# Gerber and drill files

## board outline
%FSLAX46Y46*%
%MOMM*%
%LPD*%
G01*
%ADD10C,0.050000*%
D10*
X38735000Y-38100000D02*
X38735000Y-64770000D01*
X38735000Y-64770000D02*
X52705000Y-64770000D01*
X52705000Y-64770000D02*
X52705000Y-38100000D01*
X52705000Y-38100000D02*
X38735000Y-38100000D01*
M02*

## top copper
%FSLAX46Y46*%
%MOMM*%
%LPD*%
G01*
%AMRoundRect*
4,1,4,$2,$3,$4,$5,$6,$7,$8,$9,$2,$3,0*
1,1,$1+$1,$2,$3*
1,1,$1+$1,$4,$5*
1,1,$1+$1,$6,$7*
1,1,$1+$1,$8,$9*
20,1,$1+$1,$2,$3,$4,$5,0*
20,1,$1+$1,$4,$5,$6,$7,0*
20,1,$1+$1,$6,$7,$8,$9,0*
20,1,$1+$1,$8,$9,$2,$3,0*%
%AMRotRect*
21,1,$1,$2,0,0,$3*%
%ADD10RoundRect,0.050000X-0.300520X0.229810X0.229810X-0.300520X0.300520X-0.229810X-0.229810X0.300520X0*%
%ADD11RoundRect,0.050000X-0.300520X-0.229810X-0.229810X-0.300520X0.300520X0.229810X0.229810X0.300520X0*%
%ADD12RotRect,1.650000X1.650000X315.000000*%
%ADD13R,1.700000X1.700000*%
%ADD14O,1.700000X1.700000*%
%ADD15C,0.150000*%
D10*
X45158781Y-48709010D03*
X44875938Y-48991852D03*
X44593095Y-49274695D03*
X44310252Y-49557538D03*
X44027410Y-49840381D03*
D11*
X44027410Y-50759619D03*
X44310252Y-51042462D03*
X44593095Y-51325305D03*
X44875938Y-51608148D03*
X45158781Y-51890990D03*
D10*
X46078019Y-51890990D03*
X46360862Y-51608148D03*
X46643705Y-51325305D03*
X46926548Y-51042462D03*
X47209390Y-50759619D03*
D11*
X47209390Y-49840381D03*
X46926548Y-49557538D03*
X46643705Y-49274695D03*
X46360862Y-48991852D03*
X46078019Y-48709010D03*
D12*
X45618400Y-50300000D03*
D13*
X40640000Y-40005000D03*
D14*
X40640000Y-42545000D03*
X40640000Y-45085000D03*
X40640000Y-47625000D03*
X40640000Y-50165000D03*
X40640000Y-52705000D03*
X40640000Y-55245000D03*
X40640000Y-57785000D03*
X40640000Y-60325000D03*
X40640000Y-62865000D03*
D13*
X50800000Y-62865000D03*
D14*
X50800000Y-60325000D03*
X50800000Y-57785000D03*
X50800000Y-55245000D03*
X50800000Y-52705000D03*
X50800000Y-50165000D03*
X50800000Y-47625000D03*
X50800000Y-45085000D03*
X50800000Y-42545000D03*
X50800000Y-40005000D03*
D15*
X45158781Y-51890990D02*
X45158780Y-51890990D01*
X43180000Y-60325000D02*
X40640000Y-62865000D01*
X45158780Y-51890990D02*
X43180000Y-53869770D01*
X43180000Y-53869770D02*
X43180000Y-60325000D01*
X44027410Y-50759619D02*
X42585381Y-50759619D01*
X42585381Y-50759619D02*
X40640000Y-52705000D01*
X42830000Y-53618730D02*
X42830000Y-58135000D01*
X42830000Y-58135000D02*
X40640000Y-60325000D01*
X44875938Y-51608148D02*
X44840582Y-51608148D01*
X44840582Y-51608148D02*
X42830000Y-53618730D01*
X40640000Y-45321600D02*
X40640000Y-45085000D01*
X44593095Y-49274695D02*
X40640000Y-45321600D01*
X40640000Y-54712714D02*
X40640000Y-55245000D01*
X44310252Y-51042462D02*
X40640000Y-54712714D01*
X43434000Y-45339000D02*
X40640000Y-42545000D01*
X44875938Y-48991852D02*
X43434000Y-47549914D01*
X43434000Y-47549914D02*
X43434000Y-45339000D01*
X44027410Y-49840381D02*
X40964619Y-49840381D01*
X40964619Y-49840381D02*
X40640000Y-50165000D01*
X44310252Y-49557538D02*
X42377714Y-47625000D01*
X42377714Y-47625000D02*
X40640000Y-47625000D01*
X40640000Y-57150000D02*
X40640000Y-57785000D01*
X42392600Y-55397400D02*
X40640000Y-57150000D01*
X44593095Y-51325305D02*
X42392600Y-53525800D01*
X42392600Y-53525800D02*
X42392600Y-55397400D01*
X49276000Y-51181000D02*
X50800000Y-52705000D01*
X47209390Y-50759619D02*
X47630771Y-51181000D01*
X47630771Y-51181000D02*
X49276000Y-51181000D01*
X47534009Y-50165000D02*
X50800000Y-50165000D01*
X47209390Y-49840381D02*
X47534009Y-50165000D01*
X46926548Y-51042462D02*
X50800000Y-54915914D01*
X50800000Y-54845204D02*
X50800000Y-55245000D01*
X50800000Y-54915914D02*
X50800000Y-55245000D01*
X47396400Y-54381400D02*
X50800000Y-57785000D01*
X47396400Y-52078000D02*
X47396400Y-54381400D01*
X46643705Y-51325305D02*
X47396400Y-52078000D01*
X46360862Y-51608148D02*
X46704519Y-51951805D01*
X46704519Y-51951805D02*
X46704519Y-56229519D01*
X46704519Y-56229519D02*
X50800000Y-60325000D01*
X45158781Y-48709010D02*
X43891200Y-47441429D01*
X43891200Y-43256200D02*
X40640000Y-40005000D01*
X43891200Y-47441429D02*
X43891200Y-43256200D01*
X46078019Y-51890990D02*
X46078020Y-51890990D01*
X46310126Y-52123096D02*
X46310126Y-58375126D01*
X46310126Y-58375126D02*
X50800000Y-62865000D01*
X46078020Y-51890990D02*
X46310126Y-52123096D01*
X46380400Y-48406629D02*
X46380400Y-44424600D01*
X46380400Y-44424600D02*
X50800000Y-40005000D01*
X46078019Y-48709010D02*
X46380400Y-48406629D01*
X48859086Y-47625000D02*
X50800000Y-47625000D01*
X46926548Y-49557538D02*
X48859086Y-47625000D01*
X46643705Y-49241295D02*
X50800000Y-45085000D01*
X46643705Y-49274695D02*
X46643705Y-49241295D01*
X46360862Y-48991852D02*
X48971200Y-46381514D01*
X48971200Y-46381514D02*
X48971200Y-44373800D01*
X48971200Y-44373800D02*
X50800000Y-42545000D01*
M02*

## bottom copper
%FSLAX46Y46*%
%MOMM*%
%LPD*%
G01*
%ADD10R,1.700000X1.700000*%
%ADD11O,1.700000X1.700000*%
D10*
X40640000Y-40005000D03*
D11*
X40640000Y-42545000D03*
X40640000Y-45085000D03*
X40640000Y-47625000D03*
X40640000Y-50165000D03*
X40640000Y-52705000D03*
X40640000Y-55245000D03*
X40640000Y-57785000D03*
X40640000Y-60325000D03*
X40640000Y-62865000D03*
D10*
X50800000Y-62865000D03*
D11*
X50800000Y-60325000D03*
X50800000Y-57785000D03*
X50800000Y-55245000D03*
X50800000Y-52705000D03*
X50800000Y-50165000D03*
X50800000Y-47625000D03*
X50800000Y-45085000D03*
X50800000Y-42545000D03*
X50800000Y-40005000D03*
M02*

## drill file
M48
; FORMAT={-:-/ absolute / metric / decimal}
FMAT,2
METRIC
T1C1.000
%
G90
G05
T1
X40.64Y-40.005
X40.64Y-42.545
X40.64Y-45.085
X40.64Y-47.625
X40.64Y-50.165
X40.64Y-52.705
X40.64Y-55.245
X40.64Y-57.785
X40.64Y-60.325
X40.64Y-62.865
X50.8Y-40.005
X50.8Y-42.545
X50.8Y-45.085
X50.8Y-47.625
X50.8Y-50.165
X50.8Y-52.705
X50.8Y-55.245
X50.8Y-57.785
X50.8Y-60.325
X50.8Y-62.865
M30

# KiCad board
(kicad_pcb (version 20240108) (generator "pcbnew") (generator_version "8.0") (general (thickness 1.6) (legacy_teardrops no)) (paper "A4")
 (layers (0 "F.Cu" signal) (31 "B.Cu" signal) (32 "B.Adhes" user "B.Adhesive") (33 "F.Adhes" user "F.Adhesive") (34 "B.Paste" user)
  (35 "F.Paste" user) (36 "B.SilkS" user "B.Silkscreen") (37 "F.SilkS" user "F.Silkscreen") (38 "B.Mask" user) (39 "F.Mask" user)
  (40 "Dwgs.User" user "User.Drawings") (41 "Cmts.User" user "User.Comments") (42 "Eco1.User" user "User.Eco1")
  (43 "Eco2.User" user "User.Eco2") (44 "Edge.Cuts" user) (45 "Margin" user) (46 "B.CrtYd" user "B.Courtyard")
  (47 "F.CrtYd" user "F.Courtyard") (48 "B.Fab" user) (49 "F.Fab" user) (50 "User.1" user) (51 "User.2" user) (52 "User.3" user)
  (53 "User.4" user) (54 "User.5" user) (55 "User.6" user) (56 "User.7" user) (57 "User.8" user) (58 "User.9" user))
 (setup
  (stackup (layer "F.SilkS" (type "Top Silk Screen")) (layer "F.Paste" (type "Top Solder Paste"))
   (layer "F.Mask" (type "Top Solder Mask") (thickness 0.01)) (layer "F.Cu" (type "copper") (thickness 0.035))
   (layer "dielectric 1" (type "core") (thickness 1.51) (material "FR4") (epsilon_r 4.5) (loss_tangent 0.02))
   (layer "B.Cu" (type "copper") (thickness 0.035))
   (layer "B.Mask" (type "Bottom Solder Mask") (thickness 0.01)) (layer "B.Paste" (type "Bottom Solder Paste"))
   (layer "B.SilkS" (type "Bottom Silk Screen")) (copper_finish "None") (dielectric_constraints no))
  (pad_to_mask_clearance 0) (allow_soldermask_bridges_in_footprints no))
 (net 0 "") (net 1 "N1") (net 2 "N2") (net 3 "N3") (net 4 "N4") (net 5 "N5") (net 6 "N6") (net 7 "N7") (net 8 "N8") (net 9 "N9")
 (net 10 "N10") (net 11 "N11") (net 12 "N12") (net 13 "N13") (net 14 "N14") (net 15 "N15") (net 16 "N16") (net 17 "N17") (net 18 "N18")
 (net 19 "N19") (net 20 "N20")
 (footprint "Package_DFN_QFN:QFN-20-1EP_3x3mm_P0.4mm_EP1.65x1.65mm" (layer "F.Cu") (at 45.6184 50.3 -45)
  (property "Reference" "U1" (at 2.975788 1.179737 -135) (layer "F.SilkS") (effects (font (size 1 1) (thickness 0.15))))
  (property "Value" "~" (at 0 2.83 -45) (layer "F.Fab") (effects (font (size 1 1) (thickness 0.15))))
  (pad "" smd roundrect (at -0.41 -0.41 315) (size 0.67 0.67) (layers "F.Paste") (roundrect_rratio 0.25))
  (pad "" smd roundrect (at -0.41 0.41 315) (size 0.67 0.67) (layers "F.Paste") (roundrect_rratio 0.25))
  (pad "" smd roundrect (at 0.41 -0.41 315) (size 0.67 0.67) (layers "F.Paste") (roundrect_rratio 0.25))
  (pad "" smd roundrect (at 0.41 0.41 315) (size 0.67 0.67) (layers "F.Paste") (roundrect_rratio 0.25))
  (pad "1" smd roundrect (at -1.45 -0.8 315) (size 0.85 0.2) (layers "F.Cu" "F.Paste" "F.Mask") (roundrect_rratio 0.25) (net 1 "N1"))
  (pad "2" smd roundrect (at -1.45 -0.4 315) (size 0.85 0.2) (layers "F.Cu" "F.Paste" "F.Mask") (roundrect_rratio 0.25) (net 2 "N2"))
  (pad "3" smd roundrect (at -1.45 0 315) (size 0.85 0.2) (layers "F.Cu" "F.Paste" "F.Mask") (roundrect_rratio 0.25) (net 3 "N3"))
  (pad "4" smd roundrect (at -1.45 0.4 315) (size 0.85 0.2) (layers "F.Cu" "F.Paste" "F.Mask") (roundrect_rratio 0.25) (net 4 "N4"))
  (pad "5" smd roundrect (at -1.45 0.8 315) (size 0.85 0.2) (layers "F.Cu" "F.Paste" "F.Mask") (roundrect_rratio 0.25) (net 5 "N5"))
  (pad "6" smd roundrect (at -0.8 1.45 315) (size 0.2 0.85) (layers "F.Cu" "F.Paste" "F.Mask") (roundrect_rratio 0.25) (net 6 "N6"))
  (pad "7" smd roundrect (at -0.4 1.45 315) (size 0.2 0.85) (layers "F.Cu" "F.Paste" "F.Mask") (roundrect_rratio 0.25) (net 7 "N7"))
  (pad "8" smd roundrect (at 0 1.45 315) (size 0.2 0.85) (layers "F.Cu" "F.Paste" "F.Mask") (roundrect_rratio 0.25) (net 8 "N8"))
  (pad "9" smd roundrect (at 0.4 1.45 315) (size 0.2 0.85) (layers "F.Cu" "F.Paste" "F.Mask") (roundrect_rratio 0.25) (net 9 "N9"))
  (pad "10" smd roundrect (at 0.8 1.45 315) (size 0.2 0.85) (layers "F.Cu" "F.Paste" "F.Mask") (roundrect_rratio 0.25) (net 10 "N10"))
  (pad "11" smd roundrect (at 1.45 0.8 315) (size 0.85 0.2) (layers "F.Cu" "F.Paste" "F.Mask") (roundrect_rratio 0.25) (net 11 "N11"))
  (pad "12" smd roundrect (at 1.45 0.4 315) (size 0.85 0.2) (layers "F.Cu" "F.Paste" "F.Mask") (roundrect_rratio 0.25) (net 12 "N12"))
  (pad "13" smd roundrect (at 1.45 0 315) (size 0.85 0.2) (layers "F.Cu" "F.Paste" "F.Mask") (roundrect_rratio 0.25) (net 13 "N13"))
  (pad "14" smd roundrect (at 1.45 -0.4 315) (size 0.85 0.2) (layers "F.Cu" "F.Paste" "F.Mask") (roundrect_rratio 0.25) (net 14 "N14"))
  (pad "15" smd roundrect (at 1.45 -0.8 315) (size 0.85 0.2) (layers "F.Cu" "F.Paste" "F.Mask") (roundrect_rratio 0.25) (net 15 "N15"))
  (pad "16" smd roundrect (at 0.8 -1.45 315) (size 0.2 0.85) (layers "F.Cu" "F.Paste" "F.Mask") (roundrect_rratio 0.25) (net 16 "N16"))
  (pad "17" smd roundrect (at 0.4 -1.45 315) (size 0.2 0.85) (layers "F.Cu" "F.Paste" "F.Mask") (roundrect_rratio 0.25) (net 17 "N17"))
  (pad "18" smd roundrect (at 0 -1.45 315) (size 0.2 0.85) (layers "F.Cu" "F.Paste" "F.Mask") (roundrect_rratio 0.25) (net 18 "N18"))
  (pad "19" smd roundrect (at -0.4 -1.45 315) (size 0.2 0.85) (layers "F.Cu" "F.Paste" "F.Mask") (roundrect_rratio 0.25) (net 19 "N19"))
  (pad "20" smd roundrect (at -0.8 -1.45 315) (size 0.2 0.85) (layers "F.Cu" "F.Paste" "F.Mask") (roundrect_rratio 0.25) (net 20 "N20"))
  (pad "21" smd rect (at 0 0 315) (size 1.65 1.65) (layers "F.Cu" "F.Mask") (zone_connect 2)))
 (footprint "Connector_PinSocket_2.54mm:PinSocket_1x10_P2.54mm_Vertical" (layer "B.Cu") (at 40.64 40.005 180)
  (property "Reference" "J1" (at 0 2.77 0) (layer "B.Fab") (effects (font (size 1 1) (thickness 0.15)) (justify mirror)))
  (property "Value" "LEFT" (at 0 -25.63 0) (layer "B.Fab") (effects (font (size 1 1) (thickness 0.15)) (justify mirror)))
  (pad "1" thru_hole rect (at 0 0 180) (size 1.7 1.7) (drill 1) (layers "*.Cu" "*.Mask") (remove_unused_layers no) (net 1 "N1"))
  (pad "2" thru_hole oval (at 0 -2.54 180) (size 1.7 1.7) (drill 1) (layers "*.Cu" "*.Mask") (remove_unused_layers no) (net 2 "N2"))
  (pad "3" thru_hole oval (at 0 -5.08 180) (size 1.7 1.7) (drill 1) (layers "*.Cu" "*.Mask") (remove_unused_layers no) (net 3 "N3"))
  (pad "4" thru_hole oval (at 0 -7.62 180) (size 1.7 1.7) (drill 1) (layers "*.Cu" "*.Mask") (remove_unused_layers no) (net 4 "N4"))
  (pad "5" thru_hole oval (at 0 -10.16 180) (size 1.7 1.7) (drill 1) (layers "*.Cu" "*.Mask") (remove_unused_layers no) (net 5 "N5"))
  (pad "6" thru_hole oval (at 0 -12.7 180) (size 1.7 1.7) (drill 1) (layers "*.Cu" "*.Mask") (remove_unused_layers no) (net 6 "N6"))
  (pad "7" thru_hole oval (at 0 -15.24 180) (size 1.7 1.7) (drill 1) (layers "*.Cu" "*.Mask") (remove_unused_layers no) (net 7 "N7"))
  (pad "8" thru_hole oval (at 0 -17.78 180) (size 1.7 1.7) (drill 1) (layers "*.Cu" "*.Mask") (remove_unused_layers no) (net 8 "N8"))
  (pad "9" thru_hole oval (at 0 -20.32 180) (size 1.7 1.7) (drill 1) (layers "*.Cu" "*.Mask") (remove_unused_layers no) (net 9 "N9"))
  (pad "10" thru_hole oval (at 0 -22.86 180) (size 1.7 1.7) (drill 1) (layers "*.Cu" "*.Mask") (remove_unused_layers no) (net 10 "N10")))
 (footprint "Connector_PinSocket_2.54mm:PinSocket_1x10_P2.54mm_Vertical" (layer "B.Cu") (at 50.8 62.865)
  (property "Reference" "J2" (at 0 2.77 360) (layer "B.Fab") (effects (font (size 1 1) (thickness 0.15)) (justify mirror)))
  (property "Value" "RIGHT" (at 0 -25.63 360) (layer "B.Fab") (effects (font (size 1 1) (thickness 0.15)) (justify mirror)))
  (pad "1" thru_hole rect (at 0 0) (size 1.7 1.7) (drill 1) (layers "*.Cu" "*.Mask") (remove_unused_layers no) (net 11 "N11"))
  (pad "2" thru_hole oval (at 0 -2.54) (size 1.7 1.7) (drill 1) (layers "*.Cu" "*.Mask") (remove_unused_layers no) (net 12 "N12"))
  (pad "3" thru_hole oval (at 0 -5.08) (size 1.7 1.7) (drill 1) (layers "*.Cu" "*.Mask") (remove_unused_layers no) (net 13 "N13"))
  (pad "4" thru_hole oval (at 0 -7.62) (size 1.7 1.7) (drill 1) (layers "*.Cu" "*.Mask") (remove_unused_layers no) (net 14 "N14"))
  (pad "5" thru_hole oval (at 0 -10.16) (size 1.7 1.7) (drill 1) (layers "*.Cu" "*.Mask") (remove_unused_layers no) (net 15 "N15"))
  (pad "6" thru_hole oval (at 0 -12.7) (size 1.7 1.7) (drill 1) (layers "*.Cu" "*.Mask") (remove_unused_layers no) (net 16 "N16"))
  (pad "7" thru_hole oval (at 0 -15.24) (size 1.7 1.7) (drill 1) (layers "*.Cu" "*.Mask") (remove_unused_layers no) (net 17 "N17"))
  (pad "8" thru_hole oval (at 0 -17.78) (size 1.7 1.7) (drill 1) (layers "*.Cu" "*.Mask") (remove_unused_layers no) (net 18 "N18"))
  (pad "9" thru_hole oval (at 0 -20.32) (size 1.7 1.7) (drill 1) (layers "*.Cu" "*.Mask") (remove_unused_layers no) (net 19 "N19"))
  (pad "10" thru_hole oval (at 0 -22.86) (size 1.7 1.7) (drill 1) (layers "*.Cu" "*.Mask") (remove_unused_layers no) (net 20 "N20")))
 (gr_line (start 38.735 38.1) (end 38.735 64.77) (stroke (width 0.05) (type default)) (layer "Edge.Cuts"))
 (gr_line (start 38.735 64.77) (end 52.705 64.77) (stroke (width 0.05) (type default)) (layer "Edge.Cuts"))
 (gr_line (start 52.705 64.77) (end 52.705 38.1) (stroke (width 0.05) (type default)) (layer "Edge.Cuts"))
 (gr_line (start 52.705 38.1) (end 38.735 38.1) (stroke (width 0.05) (type default)) (layer "Edge.Cuts"))
 (segment (start 45.158781 51.89099) (end 45.15878 51.89099) (width 0.15) (layer "F.Cu") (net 10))
 (segment (start 43.18 60.325) (end 40.64 62.865) (width 0.15) (layer "F.Cu") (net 10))
 (segment (start 45.15878 51.89099) (end 43.18 53.86977) (width 0.15) (layer "F.Cu") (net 10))
 (segment (start 43.18 53.86977) (end 43.18 60.325) (width 0.15) (layer "F.Cu") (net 10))
 (segment (start 44.02741 50.759619) (end 42.585381 50.759619) (width 0.15) (layer "F.Cu") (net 6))
 (segment (start 42.585381 50.759619) (end 40.64 52.705) (width 0.15) (layer "F.Cu") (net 6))
 (segment (start 42.83 53.61873) (end 42.83 58.135) (width 0.15) (layer "F.Cu") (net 9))
 (segment (start 42.83 58.135) (end 40.64 60.325) (width 0.15) (layer "F.Cu") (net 9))
 (segment (start 44.875938 51.608148) (end 44.840582 51.608148) (width 0.15) (layer "F.Cu") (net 9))
 (segment (start 44.840582 51.608148) (end 42.83 53.61873) (width 0.15) (layer "F.Cu") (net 9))
 (segment (start 40.64 45.3216) (end 40.64 45.085) (width 0.15) (layer "F.Cu") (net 3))
 (segment (start 44.593095 49.274695) (end 40.64 45.3216) (width 0.15) (layer "F.Cu") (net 3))
 (segment (start 40.64 54.712714) (end 40.64 55.245) (width 0.15) (layer "F.Cu") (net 7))
 (segment (start 44.310252 51.042462) (end 40.64 54.712714) (width 0.15) (layer "F.Cu") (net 7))
 (segment (start 43.434 45.339) (end 40.64 42.545) (width 0.15) (layer "F.Cu") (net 2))
 (segment (start 44.875938 48.991852) (end 43.434 47.549914) (width 0.15) (layer "F.Cu") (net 2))
 (segment (start 43.434 47.549914) (end 43.434 45.339) (width 0.15) (layer "F.Cu") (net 2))
 (segment (start 44.02741 49.840381) (end 40.964619 49.840381) (width 0.15) (layer "F.Cu") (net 5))
 (segment (start 40.964619 49.840381) (end 40.64 50.165) (width 0.15) (layer "F.Cu") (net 5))
 (segment (start 44.310252 49.557538) (end 42.377714 47.625) (width 0.15) (layer "F.Cu") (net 4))
 (segment (start 42.377714 47.625) (end 40.64 47.625) (width 0.15) (layer "F.Cu") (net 4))
 (segment (start 40.64 57.15) (end 40.64 57.785) (width 0.15) (layer "F.Cu") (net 8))
 (segment (start 42.3926 55.3974) (end 40.64 57.15) (width 0.15) (layer "F.Cu") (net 8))
 (segment (start 44.593095 51.325305) (end 42.3926 53.5258) (width 0.15) (layer "F.Cu") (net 8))
 (segment (start 42.3926 53.5258) (end 42.3926 55.3974) (width 0.15) (layer "F.Cu") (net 8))
 (segment (start 49.276 51.181) (end 50.8 52.705) (width 0.15) (layer "F.Cu") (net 15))
 (segment (start 47.20939 50.759619) (end 47.630771 51.181) (width 0.15) (layer "F.Cu") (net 15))
 (segment (start 47.630771 51.181) (end 49.276 51.181) (width 0.15) (layer "F.Cu") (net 15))
 (segment (start 47.534009 50.165) (end 50.8 50.165) (width 0.15) (layer "F.Cu") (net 16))
 (segment (start 47.20939 49.840381) (end 47.534009 50.165) (width 0.15) (layer "F.Cu") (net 16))
 (segment (start 46.926548 51.042462) (end 50.8 54.915914) (width 0.15) (layer "F.Cu") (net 14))
 (segment (start 50.8 54.845204) (end 50.8 55.245) (width 0.15) (layer "F.Cu") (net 14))
 (segment (start 50.8 54.915914) (end 50.8 55.245) (width 0.15) (layer "F.Cu") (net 14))
 (segment (start 47.3964 54.3814) (end 50.8 57.785) (width 0.15) (layer "F.Cu") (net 13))
 (segment (start 47.3964 52.078) (end 47.3964 54.3814) (width 0.15) (layer "F.Cu") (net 13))
 (segment (start 46.643705 51.325305) (end 47.3964 52.078) (width 0.15) (layer "F.Cu") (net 13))
 (segment (start 46.360862 51.608148) (end 46.704519 51.951805) (width 0.15) (layer "F.Cu") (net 12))
 (segment (start 46.704519 51.951805) (end 46.704519 56.229519) (width 0.15) (layer "F.Cu") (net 12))
 (segment (start 46.704519 56.229519) (end 50.8 60.325) (width 0.15) (layer "F.Cu") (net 12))
 (segment (start 45.158781 48.70901) (end 43.8912 47.441429) (width 0.15) (layer "F.Cu") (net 1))
 (segment (start 43.8912 43.2562) (end 40.64 40.005) (width 0.15) (layer "F.Cu") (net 1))
 (segment (start 43.8912 47.441429) (end 43.8912 43.2562) (width 0.15) (layer "F.Cu") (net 1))
 (segment (start 46.078019 51.89099) (end 46.07802 51.89099) (width 0.15) (layer "F.Cu") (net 11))
 (segment (start 46.310126 52.123096) (end 46.310126 58.375126) (width 0.15) (layer "F.Cu") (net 11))
 (segment (start 46.310126 58.375126) (end 50.8 62.865) (width 0.15) (layer "F.Cu") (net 11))
 (segment (start 46.07802 51.89099) (end 46.310126 52.123096) (width 0.15) (layer "F.Cu") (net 11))
 (segment (start 46.3804 48.406629) (end 46.3804 44.4246) (width 0.15) (layer "F.Cu") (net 20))
 (segment (start 46.3804 44.4246) (end 50.8 40.005) (width 0.15) (layer "F.Cu") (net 20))
 (segment (start 46.078019 48.70901) (end 46.3804 48.406629) (width 0.15) (layer "F.Cu") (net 20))
 (segment (start 48.859086 47.625) (end 50.8 47.625) (width 0.15) (layer "F.Cu") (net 17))
 (segment (start 46.926548 49.557538) (end 48.859086 47.625) (width 0.15) (layer "F.Cu") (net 17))
 (segment (start 46.643705 49.241295) (end 50.8 45.085) (width 0.15) (layer "F.Cu") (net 18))
 (segment (start 46.643705 49.274695) (end 46.643705 49.241295) (width 0.15) (layer "F.Cu") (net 18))
 (segment (start 46.360862 48.991852) (end 48.9712 46.381514) (width 0.15) (layer "F.Cu") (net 19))
 (segment (start 48.9712 46.381514) (end 48.9712 44.3738) (width 0.15) (layer "F.Cu") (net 19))
 (segment (start 48.9712 44.3738) (end 50.8 42.545) (width 0.15) (layer "F.Cu") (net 19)))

